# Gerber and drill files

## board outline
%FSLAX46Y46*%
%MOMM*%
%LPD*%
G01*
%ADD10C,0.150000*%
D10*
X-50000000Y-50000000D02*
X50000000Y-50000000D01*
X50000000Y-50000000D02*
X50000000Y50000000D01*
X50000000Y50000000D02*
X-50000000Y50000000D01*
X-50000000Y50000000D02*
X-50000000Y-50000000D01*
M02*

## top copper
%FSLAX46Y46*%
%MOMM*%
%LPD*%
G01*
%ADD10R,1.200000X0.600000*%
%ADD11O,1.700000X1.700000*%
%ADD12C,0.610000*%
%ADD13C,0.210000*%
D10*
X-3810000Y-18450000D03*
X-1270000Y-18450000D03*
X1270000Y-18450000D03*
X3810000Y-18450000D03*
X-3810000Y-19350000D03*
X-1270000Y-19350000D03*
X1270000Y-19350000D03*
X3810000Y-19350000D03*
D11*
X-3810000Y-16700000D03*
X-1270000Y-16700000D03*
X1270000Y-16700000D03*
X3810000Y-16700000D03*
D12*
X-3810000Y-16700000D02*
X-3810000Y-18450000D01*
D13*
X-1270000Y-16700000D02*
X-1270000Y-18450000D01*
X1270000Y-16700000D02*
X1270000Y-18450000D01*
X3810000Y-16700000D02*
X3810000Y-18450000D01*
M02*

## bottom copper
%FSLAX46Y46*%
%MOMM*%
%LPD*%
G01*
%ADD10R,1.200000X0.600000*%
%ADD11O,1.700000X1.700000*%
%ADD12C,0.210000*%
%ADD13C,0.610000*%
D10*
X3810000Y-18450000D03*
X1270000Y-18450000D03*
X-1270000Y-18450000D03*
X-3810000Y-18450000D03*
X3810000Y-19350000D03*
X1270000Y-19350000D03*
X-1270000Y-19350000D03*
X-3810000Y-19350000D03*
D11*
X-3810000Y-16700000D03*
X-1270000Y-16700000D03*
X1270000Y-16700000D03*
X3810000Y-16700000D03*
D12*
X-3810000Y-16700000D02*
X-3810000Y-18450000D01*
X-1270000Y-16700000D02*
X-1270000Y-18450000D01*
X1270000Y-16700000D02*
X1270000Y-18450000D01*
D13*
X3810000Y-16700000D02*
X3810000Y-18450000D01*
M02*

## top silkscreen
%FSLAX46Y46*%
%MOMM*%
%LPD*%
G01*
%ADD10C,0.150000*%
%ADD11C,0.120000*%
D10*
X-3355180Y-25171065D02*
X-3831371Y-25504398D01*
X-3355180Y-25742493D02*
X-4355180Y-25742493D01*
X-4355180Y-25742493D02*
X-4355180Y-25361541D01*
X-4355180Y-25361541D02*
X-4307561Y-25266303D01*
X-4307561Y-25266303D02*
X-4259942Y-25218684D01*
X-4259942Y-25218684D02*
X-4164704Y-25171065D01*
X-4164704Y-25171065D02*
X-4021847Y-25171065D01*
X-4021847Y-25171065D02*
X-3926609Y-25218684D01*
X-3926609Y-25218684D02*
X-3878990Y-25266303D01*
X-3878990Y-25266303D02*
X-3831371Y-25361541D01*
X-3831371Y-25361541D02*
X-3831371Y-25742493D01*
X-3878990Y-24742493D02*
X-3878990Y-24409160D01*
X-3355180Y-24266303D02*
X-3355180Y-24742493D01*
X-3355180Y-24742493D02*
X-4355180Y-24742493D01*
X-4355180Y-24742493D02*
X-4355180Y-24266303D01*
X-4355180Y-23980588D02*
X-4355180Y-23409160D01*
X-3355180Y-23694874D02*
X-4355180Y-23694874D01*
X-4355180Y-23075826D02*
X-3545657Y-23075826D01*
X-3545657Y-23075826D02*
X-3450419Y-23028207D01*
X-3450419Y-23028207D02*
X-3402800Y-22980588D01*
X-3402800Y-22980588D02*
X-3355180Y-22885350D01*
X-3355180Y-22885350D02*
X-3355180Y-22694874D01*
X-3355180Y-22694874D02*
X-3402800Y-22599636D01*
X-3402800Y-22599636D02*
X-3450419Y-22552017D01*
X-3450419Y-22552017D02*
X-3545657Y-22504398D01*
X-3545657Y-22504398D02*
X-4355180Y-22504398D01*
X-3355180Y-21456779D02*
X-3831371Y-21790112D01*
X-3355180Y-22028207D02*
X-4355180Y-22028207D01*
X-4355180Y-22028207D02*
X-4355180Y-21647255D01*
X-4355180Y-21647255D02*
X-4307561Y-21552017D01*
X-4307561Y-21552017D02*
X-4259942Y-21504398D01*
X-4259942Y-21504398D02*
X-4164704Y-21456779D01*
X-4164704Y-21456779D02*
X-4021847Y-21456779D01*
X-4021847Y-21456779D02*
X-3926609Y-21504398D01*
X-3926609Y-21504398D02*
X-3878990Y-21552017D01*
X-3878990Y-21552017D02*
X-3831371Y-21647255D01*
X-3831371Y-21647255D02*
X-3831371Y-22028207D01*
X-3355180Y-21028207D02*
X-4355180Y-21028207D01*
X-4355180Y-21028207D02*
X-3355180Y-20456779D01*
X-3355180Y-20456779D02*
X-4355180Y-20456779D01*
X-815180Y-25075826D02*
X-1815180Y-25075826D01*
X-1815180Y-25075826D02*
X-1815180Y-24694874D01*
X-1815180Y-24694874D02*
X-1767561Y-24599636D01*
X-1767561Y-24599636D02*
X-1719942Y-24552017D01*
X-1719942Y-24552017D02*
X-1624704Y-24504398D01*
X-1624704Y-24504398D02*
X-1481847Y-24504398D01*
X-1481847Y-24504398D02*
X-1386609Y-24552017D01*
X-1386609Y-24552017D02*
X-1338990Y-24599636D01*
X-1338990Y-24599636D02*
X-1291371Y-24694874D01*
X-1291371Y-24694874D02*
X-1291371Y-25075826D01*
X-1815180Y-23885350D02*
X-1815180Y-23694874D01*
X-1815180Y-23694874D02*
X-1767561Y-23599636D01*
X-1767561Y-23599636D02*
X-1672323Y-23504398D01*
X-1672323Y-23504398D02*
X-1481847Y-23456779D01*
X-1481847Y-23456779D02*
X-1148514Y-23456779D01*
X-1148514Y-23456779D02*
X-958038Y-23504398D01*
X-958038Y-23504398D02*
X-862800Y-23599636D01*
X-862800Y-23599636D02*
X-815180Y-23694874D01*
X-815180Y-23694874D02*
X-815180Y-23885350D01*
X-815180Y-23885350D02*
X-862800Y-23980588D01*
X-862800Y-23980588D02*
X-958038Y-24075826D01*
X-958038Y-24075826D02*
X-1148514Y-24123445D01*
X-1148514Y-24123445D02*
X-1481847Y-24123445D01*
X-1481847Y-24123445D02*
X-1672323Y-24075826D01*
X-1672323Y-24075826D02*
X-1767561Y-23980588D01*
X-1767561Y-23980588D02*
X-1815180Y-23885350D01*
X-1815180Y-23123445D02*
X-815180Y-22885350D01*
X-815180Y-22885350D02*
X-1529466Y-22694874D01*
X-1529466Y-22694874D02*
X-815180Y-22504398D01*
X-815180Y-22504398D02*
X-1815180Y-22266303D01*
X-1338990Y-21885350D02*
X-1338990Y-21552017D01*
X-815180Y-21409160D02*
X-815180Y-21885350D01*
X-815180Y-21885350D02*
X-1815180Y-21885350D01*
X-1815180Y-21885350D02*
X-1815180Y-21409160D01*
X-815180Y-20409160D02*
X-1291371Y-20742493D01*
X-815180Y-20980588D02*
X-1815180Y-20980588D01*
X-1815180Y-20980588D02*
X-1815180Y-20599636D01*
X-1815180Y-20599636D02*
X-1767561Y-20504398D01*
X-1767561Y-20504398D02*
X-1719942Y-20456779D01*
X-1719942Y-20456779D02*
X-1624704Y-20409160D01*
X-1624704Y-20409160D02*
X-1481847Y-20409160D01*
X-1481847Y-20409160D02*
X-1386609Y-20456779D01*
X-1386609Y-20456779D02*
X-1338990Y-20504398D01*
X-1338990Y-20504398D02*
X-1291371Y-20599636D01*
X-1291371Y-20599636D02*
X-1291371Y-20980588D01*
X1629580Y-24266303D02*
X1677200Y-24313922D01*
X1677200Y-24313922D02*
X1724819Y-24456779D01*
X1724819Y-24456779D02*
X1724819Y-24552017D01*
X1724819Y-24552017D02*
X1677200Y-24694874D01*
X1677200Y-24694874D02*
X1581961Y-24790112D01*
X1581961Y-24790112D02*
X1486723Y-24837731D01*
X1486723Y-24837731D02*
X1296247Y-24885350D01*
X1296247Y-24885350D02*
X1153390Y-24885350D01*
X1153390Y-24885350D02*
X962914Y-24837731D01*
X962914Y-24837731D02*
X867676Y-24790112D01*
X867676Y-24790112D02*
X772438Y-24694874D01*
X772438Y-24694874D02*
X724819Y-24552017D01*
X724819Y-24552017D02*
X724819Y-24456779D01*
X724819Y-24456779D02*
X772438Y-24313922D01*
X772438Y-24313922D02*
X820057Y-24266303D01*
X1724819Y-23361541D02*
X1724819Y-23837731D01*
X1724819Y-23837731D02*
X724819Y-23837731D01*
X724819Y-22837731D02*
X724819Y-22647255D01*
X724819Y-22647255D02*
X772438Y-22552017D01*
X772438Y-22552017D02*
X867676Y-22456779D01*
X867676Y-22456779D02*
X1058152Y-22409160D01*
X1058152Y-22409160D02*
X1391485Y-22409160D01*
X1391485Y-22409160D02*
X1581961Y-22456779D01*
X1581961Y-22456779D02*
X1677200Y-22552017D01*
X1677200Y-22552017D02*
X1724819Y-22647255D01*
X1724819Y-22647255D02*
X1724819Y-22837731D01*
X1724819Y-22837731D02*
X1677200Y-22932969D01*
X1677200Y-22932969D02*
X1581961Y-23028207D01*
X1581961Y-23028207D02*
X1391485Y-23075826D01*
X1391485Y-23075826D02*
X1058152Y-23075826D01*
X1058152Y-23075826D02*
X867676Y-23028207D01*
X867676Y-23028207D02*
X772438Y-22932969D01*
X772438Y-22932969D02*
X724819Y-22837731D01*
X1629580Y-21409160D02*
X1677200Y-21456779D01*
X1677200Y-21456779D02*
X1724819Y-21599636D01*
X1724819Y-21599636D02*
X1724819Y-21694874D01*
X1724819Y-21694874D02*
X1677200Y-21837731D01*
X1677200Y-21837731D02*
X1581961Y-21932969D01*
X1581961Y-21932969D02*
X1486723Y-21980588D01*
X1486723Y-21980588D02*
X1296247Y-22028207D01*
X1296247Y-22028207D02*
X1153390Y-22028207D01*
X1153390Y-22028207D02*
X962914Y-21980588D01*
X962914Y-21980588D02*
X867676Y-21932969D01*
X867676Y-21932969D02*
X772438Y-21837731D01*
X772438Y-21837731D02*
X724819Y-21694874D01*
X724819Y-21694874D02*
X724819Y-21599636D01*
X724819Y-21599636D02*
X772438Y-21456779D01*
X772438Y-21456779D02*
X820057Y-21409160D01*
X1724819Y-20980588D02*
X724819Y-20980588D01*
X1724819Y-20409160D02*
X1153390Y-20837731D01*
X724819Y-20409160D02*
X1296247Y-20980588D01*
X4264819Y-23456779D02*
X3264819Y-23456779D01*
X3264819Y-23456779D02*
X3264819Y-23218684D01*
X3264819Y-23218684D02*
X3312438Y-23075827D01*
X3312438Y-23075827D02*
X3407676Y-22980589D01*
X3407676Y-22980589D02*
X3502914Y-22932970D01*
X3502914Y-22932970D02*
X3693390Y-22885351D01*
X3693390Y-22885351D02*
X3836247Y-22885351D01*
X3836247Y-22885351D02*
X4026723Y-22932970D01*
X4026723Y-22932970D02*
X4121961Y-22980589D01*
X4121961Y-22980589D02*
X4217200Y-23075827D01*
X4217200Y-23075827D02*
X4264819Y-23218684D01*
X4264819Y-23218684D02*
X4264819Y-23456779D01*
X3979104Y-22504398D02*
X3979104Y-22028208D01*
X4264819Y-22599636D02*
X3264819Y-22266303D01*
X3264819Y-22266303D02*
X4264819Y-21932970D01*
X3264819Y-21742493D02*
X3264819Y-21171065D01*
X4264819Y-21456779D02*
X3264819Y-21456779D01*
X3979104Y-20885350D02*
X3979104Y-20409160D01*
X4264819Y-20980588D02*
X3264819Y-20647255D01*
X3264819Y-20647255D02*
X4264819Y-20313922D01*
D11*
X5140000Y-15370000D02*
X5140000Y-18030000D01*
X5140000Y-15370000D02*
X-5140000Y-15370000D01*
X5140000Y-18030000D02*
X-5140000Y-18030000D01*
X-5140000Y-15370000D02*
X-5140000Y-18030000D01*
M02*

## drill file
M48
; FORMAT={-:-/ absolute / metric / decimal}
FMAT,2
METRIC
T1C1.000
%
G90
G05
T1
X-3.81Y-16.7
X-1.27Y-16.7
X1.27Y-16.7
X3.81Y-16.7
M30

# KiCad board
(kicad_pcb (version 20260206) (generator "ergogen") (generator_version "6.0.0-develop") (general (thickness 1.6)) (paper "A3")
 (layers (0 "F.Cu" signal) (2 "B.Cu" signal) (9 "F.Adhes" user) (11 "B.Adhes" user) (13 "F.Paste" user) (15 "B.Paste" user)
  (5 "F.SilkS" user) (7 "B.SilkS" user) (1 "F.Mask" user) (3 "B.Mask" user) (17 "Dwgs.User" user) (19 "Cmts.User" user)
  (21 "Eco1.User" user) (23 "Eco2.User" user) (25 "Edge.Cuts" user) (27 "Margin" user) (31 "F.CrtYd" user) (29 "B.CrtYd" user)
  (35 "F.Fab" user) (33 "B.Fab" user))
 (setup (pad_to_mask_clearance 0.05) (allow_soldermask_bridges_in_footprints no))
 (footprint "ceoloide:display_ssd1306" (layer "F.Cu") (at 0 0 0)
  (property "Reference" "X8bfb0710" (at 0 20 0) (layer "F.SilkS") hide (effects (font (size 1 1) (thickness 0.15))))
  (fp_line (start 5.14 15.37) (end 5.14 18.03) (layer "F.SilkS") (stroke (width 0.12) (type solid)))
  (fp_line (start 5.14 15.37) (end -5.14 15.37) (layer "F.SilkS") (stroke (width 0.12) (type solid)))
  (fp_line (start 5.14 18.03) (end -5.14 18.03) (layer "F.SilkS") (stroke (width 0.12) (type solid)))
  (fp_line (start -5.14 15.37) (end -5.14 18.03) (layer "F.SilkS") (stroke (width 0.12) (type solid)))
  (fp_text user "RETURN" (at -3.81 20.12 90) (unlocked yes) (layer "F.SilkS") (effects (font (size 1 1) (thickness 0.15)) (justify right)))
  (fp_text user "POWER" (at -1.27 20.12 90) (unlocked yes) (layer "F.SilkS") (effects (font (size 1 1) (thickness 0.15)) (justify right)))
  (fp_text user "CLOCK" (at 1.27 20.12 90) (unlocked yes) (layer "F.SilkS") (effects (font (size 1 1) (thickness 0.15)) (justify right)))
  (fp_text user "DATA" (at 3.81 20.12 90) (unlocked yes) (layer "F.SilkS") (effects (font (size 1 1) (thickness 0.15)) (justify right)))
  (pad "14" smd rect (at -3.81 18.450000000000003 90) (size 0.6 1.2) (layers "F.Cu" "F.Paste" "F.Mask") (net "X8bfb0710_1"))
  (pad "15" smd rect (at -1.27 18.450000000000003 90) (size 0.6 1.2) (layers "F.Cu" "F.Paste" "F.Mask") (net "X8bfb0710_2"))
  (pad "16" smd rect (at 1.27 18.450000000000003 90) (size 0.6 1.2) (layers "F.Cu" "F.Paste" "F.Mask") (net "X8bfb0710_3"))
  (pad "17" smd rect (at 3.81 18.450000000000003 90) (size 0.6 1.2) (layers "F.Cu" "F.Paste" "F.Mask") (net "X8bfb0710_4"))
  (pad "10" smd rect (at -3.81 19.35 90) (size 0.6 1.2) (layers "F.Cu" "F.Paste" "F.Mask") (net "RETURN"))
  (pad "11" smd rect (at -1.27 19.35 90) (size 0.6 1.2) (layers "F.Cu" "F.Paste" "F.Mask") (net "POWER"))
  (pad "12" smd rect (at 1.27 19.35 90) (size 0.6 1.2) (layers "F.Cu" "F.Paste" "F.Mask") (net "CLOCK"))
  (pad "13" smd rect (at 3.81 19.35 90) (size 0.6 1.2) (layers "F.Cu" "F.Paste" "F.Mask") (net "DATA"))
  (pad "24" smd rect (at 3.81 18.450000000000003 270) (size 0.6 1.2) (layers "B.Cu" "B.Paste" "B.Mask") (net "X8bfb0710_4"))
  (pad "25" smd rect (at 1.27 18.450000000000003 270) (size 0.6 1.2) (layers "B.Cu" "B.Paste" "B.Mask") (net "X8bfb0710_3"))
  (pad "26" smd rect (at -1.27 18.450000000000003 270) (size 0.6 1.2) (layers "B.Cu" "B.Paste" "B.Mask") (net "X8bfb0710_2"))
  (pad "27" smd rect (at -3.81 18.450000000000003 270) (size 0.6 1.2) (layers "B.Cu" "B.Paste" "B.Mask") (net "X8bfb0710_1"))
  (pad "20" smd rect (at 3.81 19.35 270) (size 0.6 1.2) (layers "B.Cu" "B.Paste" "B.Mask") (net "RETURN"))
  (pad "21" smd rect (at 1.27 19.35 270) (size 0.6 1.2) (layers "B.Cu" "B.Paste" "B.Mask") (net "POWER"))
  (pad "22" smd rect (at -1.27 19.35 270) (size 0.6 1.2) (layers "B.Cu" "B.Paste" "B.Mask") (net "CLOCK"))
  (pad "23" smd rect (at -3.81 19.35 270) (size 0.6 1.2) (layers "B.Cu" "B.Paste" "B.Mask") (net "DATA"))
  (pad "1" thru_hole oval (at -3.81 16.7 270) (size 1.7 1.7) (drill 1) (layers "*.Cu" "*.Mask") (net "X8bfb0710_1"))
  (pad "2" thru_hole oval (at -1.27 16.7 270) (size 1.7 1.7) (drill 1) (layers "*.Cu" "*.Mask") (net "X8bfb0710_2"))
  (pad "3" thru_hole oval (at 1.27 16.7 270) (size 1.7 1.7) (drill 1) (layers "*.Cu" "*.Mask") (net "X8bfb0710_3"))
  (pad "4" thru_hole oval (at 3.81 16.7 270) (size 1.7 1.7) (drill 1) (layers "*.Cu" "*.Mask") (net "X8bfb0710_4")))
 (segment (start -3.81 16.7) (end -3.81 18.45) (width 0.61) (layer "F.Cu") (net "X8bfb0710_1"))
 (segment (start -1.27 16.7) (end -1.27 18.45) (width 0.21) (layer "F.Cu") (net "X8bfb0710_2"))
 (segment (start 1.27 16.7) (end 1.27 18.45) (width 0.21) (layer "F.Cu") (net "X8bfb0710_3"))
 (segment (start 3.81 16.7) (end 3.81 18.45) (width 0.21) (layer "F.Cu") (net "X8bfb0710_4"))
 (segment (start -3.81 16.7) (end -3.81 18.45) (width 0.21) (layer "B.Cu") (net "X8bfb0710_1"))
 (segment (start -1.27 16.7) (end -1.27 18.45) (width 0.21) (layer "B.Cu") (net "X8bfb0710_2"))
 (segment (start 1.27 16.7) (end 1.27 18.45) (width 0.21) (layer "B.Cu") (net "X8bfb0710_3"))
 (segment (start 3.81 16.7) (end 3.81 18.45) (width 0.61) (layer "B.Cu") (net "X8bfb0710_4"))
 (gr_line (start -50 50) (end 50 50) (layer Edge.Cuts) (stroke (width 0.15) (type default)))
 (gr_line (start 50 50) (end 50 -50) (layer Edge.Cuts) (stroke (width 0.15) (type default)))
 (gr_line (start 50 -50) (end -50 -50) (layer Edge.Cuts) (stroke (width 0.15) (type default)))
 (gr_line (start -50 -50) (end -50 50) (layer Edge.Cuts) (stroke (width 0.15) (type default))))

